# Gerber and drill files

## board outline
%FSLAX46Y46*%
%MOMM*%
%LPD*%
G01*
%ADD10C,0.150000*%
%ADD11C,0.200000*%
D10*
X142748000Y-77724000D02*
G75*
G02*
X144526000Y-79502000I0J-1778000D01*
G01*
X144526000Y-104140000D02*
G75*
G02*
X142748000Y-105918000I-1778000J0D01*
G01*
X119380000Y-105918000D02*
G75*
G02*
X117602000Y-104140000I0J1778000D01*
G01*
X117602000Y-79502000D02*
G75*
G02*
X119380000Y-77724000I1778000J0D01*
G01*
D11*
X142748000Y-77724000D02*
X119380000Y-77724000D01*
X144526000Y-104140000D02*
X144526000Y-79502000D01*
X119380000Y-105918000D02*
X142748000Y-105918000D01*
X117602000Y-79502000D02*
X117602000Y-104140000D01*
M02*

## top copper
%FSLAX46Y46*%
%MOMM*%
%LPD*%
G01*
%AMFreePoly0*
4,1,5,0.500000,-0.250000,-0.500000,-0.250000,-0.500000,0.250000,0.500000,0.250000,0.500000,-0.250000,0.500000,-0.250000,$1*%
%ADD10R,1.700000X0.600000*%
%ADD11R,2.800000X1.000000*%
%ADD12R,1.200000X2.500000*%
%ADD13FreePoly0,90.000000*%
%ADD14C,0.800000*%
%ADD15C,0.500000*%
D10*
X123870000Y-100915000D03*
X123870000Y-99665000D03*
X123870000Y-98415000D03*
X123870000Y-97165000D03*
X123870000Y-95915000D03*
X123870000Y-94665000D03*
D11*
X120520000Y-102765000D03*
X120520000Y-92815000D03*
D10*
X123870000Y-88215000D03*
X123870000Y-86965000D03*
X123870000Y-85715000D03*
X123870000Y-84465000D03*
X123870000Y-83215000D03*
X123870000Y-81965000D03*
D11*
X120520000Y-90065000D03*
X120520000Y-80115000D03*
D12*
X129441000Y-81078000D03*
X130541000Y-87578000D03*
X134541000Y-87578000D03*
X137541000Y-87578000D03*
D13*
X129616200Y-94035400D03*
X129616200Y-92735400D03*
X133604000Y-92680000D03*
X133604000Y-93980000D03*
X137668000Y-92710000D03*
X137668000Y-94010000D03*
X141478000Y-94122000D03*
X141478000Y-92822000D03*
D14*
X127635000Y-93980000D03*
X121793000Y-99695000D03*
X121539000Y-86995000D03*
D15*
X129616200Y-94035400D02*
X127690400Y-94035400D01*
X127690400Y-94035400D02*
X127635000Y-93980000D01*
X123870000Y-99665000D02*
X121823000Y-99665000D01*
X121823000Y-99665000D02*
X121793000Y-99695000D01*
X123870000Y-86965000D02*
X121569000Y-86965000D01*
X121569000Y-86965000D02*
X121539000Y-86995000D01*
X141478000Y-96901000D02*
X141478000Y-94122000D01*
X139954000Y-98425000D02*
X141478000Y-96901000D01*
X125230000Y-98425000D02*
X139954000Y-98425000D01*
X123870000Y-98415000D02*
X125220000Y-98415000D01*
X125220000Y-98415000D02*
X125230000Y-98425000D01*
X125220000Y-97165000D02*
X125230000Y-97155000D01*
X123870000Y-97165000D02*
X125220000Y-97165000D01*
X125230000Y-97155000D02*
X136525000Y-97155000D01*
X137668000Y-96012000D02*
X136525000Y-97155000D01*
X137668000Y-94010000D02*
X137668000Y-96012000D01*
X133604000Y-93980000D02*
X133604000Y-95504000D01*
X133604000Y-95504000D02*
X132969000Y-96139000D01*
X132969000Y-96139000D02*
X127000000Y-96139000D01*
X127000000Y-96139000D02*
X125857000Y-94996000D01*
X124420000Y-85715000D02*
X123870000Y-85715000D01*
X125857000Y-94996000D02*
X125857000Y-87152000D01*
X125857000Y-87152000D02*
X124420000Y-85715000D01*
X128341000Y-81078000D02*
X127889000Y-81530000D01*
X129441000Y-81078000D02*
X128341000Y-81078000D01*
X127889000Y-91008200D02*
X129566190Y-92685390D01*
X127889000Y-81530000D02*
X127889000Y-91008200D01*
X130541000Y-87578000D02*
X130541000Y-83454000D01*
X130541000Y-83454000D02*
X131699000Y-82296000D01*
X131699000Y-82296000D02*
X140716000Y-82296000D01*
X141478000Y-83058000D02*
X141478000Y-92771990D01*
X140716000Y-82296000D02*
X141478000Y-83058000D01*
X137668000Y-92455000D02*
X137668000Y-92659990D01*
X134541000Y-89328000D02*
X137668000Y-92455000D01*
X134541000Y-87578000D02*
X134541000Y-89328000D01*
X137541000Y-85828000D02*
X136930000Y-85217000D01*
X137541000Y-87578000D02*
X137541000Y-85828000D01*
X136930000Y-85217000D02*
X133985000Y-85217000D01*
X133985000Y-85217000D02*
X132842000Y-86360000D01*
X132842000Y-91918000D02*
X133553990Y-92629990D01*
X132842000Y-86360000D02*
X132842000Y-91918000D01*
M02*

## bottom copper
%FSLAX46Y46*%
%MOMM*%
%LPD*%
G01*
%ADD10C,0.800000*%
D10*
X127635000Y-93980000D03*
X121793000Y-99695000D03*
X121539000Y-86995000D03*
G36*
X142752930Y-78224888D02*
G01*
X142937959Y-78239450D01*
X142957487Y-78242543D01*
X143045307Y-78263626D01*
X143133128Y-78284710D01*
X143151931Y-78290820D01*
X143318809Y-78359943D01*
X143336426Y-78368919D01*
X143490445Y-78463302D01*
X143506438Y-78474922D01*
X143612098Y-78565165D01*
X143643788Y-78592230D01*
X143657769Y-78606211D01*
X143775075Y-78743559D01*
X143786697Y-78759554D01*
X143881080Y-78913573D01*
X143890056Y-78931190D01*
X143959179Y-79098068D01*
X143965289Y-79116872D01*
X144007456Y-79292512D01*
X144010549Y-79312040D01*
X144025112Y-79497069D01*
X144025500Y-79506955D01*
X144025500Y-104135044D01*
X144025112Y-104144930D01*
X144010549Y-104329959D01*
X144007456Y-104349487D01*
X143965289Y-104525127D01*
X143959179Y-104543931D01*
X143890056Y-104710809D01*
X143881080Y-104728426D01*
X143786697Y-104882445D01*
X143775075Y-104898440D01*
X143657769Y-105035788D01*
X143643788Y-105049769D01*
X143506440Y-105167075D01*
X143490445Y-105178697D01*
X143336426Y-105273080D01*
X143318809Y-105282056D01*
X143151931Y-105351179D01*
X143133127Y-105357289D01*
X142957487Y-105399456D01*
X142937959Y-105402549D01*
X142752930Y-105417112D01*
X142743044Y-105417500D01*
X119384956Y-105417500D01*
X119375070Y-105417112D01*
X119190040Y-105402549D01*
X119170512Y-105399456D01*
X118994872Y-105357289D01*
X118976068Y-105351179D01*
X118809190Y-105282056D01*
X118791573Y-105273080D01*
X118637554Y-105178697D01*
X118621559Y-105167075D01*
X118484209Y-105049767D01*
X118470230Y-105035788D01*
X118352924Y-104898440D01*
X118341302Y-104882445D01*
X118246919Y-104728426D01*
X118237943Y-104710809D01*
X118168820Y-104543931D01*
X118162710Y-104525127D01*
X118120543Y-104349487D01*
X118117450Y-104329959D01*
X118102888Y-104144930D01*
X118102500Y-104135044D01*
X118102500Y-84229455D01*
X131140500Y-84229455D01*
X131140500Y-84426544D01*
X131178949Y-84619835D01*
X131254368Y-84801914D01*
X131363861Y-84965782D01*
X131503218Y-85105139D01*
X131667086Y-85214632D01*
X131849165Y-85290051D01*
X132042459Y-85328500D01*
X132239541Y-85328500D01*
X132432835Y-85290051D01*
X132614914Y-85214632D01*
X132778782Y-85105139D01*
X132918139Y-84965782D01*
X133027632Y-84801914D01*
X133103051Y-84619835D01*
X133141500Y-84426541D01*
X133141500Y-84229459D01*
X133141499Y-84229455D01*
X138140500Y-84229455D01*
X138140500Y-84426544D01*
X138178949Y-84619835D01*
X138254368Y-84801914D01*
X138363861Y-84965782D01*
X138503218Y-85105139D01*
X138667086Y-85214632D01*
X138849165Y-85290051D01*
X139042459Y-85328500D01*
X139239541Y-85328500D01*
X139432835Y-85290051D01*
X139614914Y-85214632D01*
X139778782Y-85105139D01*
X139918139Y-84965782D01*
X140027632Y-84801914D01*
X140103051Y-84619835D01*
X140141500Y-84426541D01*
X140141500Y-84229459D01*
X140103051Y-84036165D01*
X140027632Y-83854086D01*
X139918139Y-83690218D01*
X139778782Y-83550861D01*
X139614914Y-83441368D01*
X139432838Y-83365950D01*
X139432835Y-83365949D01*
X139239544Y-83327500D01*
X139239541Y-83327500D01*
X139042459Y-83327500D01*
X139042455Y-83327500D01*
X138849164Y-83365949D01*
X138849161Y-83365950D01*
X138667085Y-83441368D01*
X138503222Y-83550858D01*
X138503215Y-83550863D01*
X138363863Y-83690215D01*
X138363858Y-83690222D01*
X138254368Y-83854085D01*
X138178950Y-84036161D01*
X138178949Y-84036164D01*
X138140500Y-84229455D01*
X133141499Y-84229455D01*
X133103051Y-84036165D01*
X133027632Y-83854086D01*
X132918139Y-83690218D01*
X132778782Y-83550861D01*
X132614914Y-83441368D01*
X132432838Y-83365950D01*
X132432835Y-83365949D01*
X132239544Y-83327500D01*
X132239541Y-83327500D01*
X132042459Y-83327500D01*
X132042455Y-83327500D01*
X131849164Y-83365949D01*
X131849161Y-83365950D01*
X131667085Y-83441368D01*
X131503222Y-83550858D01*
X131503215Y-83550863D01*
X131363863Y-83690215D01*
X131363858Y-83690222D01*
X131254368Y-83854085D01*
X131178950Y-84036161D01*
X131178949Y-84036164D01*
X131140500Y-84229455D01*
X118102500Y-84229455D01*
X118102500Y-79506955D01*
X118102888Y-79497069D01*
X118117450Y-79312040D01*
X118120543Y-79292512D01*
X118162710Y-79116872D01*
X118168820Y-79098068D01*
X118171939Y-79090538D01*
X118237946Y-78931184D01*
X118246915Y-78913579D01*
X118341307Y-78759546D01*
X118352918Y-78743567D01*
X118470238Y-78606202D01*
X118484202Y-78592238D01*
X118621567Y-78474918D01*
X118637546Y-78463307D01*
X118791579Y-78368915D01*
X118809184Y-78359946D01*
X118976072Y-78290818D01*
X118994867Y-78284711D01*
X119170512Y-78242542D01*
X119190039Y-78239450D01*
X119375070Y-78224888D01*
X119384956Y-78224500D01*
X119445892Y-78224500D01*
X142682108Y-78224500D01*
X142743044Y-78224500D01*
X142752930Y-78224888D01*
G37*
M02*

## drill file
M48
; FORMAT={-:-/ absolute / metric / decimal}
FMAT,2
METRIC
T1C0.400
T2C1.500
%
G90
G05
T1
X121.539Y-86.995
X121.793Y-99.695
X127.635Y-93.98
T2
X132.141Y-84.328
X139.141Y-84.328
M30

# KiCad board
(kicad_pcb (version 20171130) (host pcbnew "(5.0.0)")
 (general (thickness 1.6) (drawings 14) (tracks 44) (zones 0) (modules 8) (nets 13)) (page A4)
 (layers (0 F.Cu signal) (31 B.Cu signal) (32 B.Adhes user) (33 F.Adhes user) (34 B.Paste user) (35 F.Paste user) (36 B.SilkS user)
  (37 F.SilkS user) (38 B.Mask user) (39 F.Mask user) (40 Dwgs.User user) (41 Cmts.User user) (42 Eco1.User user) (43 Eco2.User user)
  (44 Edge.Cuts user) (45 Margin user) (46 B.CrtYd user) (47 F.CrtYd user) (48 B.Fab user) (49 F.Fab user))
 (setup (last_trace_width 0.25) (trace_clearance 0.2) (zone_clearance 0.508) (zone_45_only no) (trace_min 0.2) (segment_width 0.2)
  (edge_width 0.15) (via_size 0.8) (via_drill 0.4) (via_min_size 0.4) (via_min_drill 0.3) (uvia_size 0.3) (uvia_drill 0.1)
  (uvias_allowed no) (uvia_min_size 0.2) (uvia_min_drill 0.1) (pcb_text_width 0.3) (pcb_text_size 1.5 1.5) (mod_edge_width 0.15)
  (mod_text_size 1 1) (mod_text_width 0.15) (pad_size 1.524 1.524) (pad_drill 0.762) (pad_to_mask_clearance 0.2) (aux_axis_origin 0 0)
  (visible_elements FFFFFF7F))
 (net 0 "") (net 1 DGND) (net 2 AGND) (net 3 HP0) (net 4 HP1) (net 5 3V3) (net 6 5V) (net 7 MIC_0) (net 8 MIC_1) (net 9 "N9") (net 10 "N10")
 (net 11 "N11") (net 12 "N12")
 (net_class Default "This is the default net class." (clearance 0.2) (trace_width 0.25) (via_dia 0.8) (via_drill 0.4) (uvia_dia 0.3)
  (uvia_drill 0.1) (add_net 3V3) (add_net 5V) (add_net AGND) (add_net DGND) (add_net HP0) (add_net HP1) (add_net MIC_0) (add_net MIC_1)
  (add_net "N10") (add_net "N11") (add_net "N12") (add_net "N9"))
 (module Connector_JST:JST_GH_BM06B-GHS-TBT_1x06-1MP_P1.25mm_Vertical (layer F.Cu) (at 121.92 97.79 90)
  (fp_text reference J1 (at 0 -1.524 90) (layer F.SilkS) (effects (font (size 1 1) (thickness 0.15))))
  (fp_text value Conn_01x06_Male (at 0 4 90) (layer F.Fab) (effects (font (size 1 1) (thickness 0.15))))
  (pad 1 smd rect (at -3.125 1.95 90) (size 0.6 1.7) (layers F.Cu F.Paste F.Mask) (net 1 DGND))
  (pad 2 smd rect (at -1.875 1.95 90) (size 0.6 1.7) (layers F.Cu F.Paste F.Mask) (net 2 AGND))
  (pad 3 smd rect (at -0.625 1.95 90) (size 0.6 1.7) (layers F.Cu F.Paste F.Mask) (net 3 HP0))
  (pad 4 smd rect (at 0.625 1.95 90) (size 0.6 1.7) (layers F.Cu F.Paste F.Mask) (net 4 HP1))
  (pad 5 smd rect (at 1.875 1.95 90) (size 0.6 1.7) (layers F.Cu F.Paste F.Mask) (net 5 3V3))
  (pad 6 smd rect (at 3.125 1.95 90) (size 0.6 1.7) (layers F.Cu F.Paste F.Mask) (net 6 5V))
  (pad MP smd rect (at -4.975 -1.4 90) (size 1 2.8) (layers F.Cu F.Paste F.Mask))
  (pad MP smd rect (at 4.975 -1.4 90) (size 1 2.8) (layers F.Cu F.Paste F.Mask)))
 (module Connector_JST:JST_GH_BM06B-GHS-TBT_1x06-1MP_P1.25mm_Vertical (layer F.Cu) (at 121.92 85.09 90)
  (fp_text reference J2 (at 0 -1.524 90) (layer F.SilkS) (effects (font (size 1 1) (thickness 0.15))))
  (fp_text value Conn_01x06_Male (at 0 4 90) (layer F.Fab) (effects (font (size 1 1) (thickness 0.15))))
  (pad 1 smd rect (at -3.125 1.95 90) (size 0.6 1.7) (layers F.Cu F.Paste F.Mask) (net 1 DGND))
  (pad 2 smd rect (at -1.875 1.95 90) (size 0.6 1.7) (layers F.Cu F.Paste F.Mask) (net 2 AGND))
  (pad 3 smd rect (at -0.625 1.95 90) (size 0.6 1.7) (layers F.Cu F.Paste F.Mask) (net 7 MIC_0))
  (pad 4 smd rect (at 0.625 1.95 90) (size 0.6 1.7) (layers F.Cu F.Paste F.Mask) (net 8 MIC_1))
  (pad 5 smd rect (at 1.875 1.95 90) (size 0.6 1.7) (layers F.Cu F.Paste F.Mask) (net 5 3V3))
  (pad 6 smd rect (at 3.125 1.95 90) (size 0.6 1.7) (layers F.Cu F.Paste F.Mask) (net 6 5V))
  (pad MP smd rect (at -4.975 -1.4 90) (size 1 2.8) (layers F.Cu F.Paste F.Mask))
  (pad MP smd rect (at 4.975 -1.4 90) (size 1 2.8) (layers F.Cu F.Paste F.Mask)))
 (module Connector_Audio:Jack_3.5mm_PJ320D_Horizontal (layer F.Cu) (at 134.366 84.328 180)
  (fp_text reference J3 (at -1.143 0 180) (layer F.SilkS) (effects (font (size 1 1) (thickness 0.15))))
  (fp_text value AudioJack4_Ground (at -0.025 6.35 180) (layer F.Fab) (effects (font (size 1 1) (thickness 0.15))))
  (pad 4 smd rect (at 4.925 3.25 180) (size 1.2 2.5) (layers F.Cu F.Paste F.Mask) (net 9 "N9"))
  (pad 1 smd rect (at 3.825 -3.25 180) (size 1.2 2.5) (layers F.Cu F.Paste F.Mask) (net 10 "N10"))
  (pad 2 smd rect (at -0.175 -3.25 180) (size 1.2 2.5) (layers F.Cu F.Paste F.Mask) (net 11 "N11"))
  (pad 3 smd rect (at -3.175 -3.25 180) (size 1.2 2.5) (layers F.Cu F.Paste F.Mask) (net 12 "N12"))
  (pad "" np_thru_hole circle (at -4.775 0 180) (size 1.5 1.5) (drill 1.5) (layers *.Cu *.Mask))
  (pad "" np_thru_hole circle (at 2.225 0 180) (size 1.5 1.5) (drill 1.5) (layers *.Cu *.Mask)))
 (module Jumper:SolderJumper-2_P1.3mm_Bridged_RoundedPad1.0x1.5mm (layer F.Cu) (at 129.6162 93.3854 90)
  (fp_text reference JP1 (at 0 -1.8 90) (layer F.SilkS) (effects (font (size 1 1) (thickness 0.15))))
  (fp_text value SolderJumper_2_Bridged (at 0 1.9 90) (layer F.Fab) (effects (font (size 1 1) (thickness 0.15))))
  (pad 1 smd custom (at -0.65 0 90) (size 1 0.5) (layers F.Cu F.Mask) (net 2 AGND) (zone_connect 0)
   (options (clearance outline) (anchor rect)) (primitives))
  (pad 2 smd custom (at 0.65 0 90) (size 1 0.5) (layers F.Cu F.Mask) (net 9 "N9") (zone_connect 0)
   (options (clearance outline) (anchor rect)) (primitives)))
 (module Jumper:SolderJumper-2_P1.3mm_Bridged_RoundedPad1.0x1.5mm (layer F.Cu) (at 133.604 93.33 90)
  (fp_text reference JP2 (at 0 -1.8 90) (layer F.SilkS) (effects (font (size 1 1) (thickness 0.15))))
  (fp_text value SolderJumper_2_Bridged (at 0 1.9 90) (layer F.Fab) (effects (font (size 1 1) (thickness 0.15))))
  (pad 2 smd custom (at 0.65 0 90) (size 1 0.5) (layers F.Cu F.Mask) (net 12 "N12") (zone_connect 0)
   (options (clearance outline) (anchor rect)) (primitives))
  (pad 1 smd custom (at -0.65 0 90) (size 1 0.5) (layers F.Cu F.Mask) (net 7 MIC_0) (zone_connect 0)
   (options (clearance outline) (anchor rect)) (primitives)))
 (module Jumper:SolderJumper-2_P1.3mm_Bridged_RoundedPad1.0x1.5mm (layer F.Cu) (at 137.668 93.36 90)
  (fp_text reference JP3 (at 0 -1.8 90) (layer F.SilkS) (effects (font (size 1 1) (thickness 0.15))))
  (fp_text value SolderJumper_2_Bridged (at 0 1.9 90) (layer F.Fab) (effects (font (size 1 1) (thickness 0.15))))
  (pad 2 smd custom (at 0.65 0 90) (size 1 0.5) (layers F.Cu F.Mask) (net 11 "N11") (zone_connect 0)
   (options (clearance outline) (anchor rect)) (primitives))
  (pad 1 smd custom (at -0.65 0 90) (size 1 0.5) (layers F.Cu F.Mask) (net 4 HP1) (zone_connect 0)
   (options (clearance outline) (anchor rect)) (primitives)))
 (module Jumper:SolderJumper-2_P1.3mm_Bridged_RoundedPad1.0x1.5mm (layer F.Cu) (at 141.478 93.472 90)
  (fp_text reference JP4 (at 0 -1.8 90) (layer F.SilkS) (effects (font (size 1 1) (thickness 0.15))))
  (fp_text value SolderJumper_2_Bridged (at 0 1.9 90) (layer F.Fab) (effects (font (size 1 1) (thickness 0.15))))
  (pad 1 smd custom (at -0.65 0 90) (size 1 0.5) (layers F.Cu F.Mask) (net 3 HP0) (zone_connect 0)
   (options (clearance outline) (anchor rect)) (primitives))
  (pad 2 smd custom (at 0.65 0 90) (size 1 0.5) (layers F.Cu F.Mask) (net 10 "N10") (zone_connect 0)
   (options (clearance outline) (anchor rect)) (primitives)))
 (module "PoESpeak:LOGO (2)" (layer F.Cu) (at 135.128 102.616)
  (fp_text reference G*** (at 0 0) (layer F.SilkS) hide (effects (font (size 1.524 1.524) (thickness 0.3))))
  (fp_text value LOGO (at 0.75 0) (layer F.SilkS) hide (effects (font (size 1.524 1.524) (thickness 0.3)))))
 (gr_arc (start 142.748 79.502) (end 144.526 79.502) (angle -90) (layer Edge.Cuts) (width 0.15))
 (gr_arc (start 142.748 104.14) (end 142.748 105.918) (angle -90) (layer Edge.Cuts) (width 0.15))
 (gr_arc (start 119.38 104.14) (end 117.602 104.14) (angle -90) (layer Edge.Cuts) (width 0.15))
 (gr_arc (start 119.38 79.502) (end 119.38 77.724) (angle -90) (layer Edge.Cuts) (width 0.15))
 (gr_line (start 142.748 77.724) (end 119.38 77.724) (layer Edge.Cuts) (width 0.2))
 (gr_line (start 144.526 104.14) (end 144.526 79.502) (layer Edge.Cuts) (width 0.2))
 (gr_line (start 119.38 105.918) (end 142.748 105.918) (layer Edge.Cuts) (width 0.2))
 (gr_line (start 117.602 79.502) (end 117.602 104.14) (layer Edge.Cuts) (width 0.2))
 (via (at 127.635 93.98) (size 0.8) (drill 0.4) (layers F.Cu B.Cu) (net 2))
 (segment (start 129.6162 94.0354) (end 127.6904 94.0354) (width 0.5) (layer F.Cu) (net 2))
 (segment (start 127.6904 94.0354) (end 127.635 93.98) (width 0.5) (layer F.Cu) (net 2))
 (via (at 121.793 99.695) (size 0.8) (drill 0.4) (layers F.Cu B.Cu) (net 2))
 (segment (start 123.87 99.665) (end 121.823 99.665) (width 0.5) (layer F.Cu) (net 2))
 (segment (start 121.823 99.665) (end 121.793 99.695) (width 0.5) (layer F.Cu) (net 2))
 (via (at 121.539 86.995) (size 0.8) (drill 0.4) (layers F.Cu B.Cu) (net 2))
 (segment (start 123.87 86.965) (end 121.569 86.965) (width 0.5) (layer F.Cu) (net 2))
 (segment (start 121.569 86.965) (end 121.539 86.995) (width 0.5) (layer F.Cu) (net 2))
 (segment (start 141.478 96.901) (end 141.478 94.122) (width 0.5) (layer F.Cu) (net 3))
 (segment (start 139.954 98.425) (end 141.478 96.901) (width 0.5) (layer F.Cu) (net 3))
 (segment (start 125.23 98.425) (end 139.954 98.425) (width 0.5) (layer F.Cu) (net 3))
 (segment (start 123.87 98.415) (end 125.22 98.415) (width 0.5) (layer F.Cu) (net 3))
 (segment (start 125.22 98.415) (end 125.23 98.425) (width 0.5) (layer F.Cu) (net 3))
 (segment (start 125.22 97.165) (end 125.23 97.155) (width 0.5) (layer F.Cu) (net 4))
 (segment (start 123.87 97.165) (end 125.22 97.165) (width 0.5) (layer F.Cu) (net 4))
 (segment (start 125.23 97.155) (end 136.525 97.155) (width 0.5) (layer F.Cu) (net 4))
 (segment (start 137.668 96.012) (end 136.525 97.155) (width 0.5) (layer F.Cu) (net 4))
 (segment (start 137.668 94.01) (end 137.668 96.012) (width 0.5) (layer F.Cu) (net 4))
 (segment (start 133.604 93.98) (end 133.604 95.504) (width 0.5) (layer F.Cu) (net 7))
 (segment (start 133.604 95.504) (end 132.969 96.139) (width 0.5) (layer F.Cu) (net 7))
 (segment (start 132.969 96.139) (end 127 96.139) (width 0.5) (layer F.Cu) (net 7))
 (segment (start 127 96.139) (end 125.857 94.996) (width 0.5) (layer F.Cu) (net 7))
 (segment (start 124.42 85.715) (end 123.87 85.715) (width 0.5) (layer F.Cu) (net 7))
 (segment (start 125.857 94.996) (end 125.857 87.152) (width 0.5) (layer F.Cu) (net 7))
 (segment (start 125.857 87.152) (end 124.42 85.715) (width 0.5) (layer F.Cu) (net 7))
 (segment (start 128.341 81.078) (end 127.889 81.53) (width 0.5) (layer F.Cu) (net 9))
 (segment (start 129.441 81.078) (end 128.341 81.078) (width 0.5) (layer F.Cu) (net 9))
 (segment (start 127.889 91.0082) (end 129.56619 92.68539) (width 0.5) (layer F.Cu) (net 9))
 (segment (start 127.889 81.53) (end 127.889 91.0082) (width 0.5) (layer F.Cu) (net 9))
 (segment (start 130.541 87.578) (end 130.541 83.454) (width 0.5) (layer F.Cu) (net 10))
 (segment (start 130.541 83.454) (end 131.699 82.296) (width 0.5) (layer F.Cu) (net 10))
 (segment (start 131.699 82.296) (end 140.716 82.296) (width 0.5) (layer F.Cu) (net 10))
 (segment (start 141.478 83.058) (end 141.478 92.77199) (width 0.5) (layer F.Cu) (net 10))
 (segment (start 140.716 82.296) (end 141.478 83.058) (width 0.5) (layer F.Cu) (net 10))
 (segment (start 137.668 92.455) (end 137.668 92.65999) (width 0.5) (layer F.Cu) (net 11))
 (segment (start 134.541 89.328) (end 137.668 92.455) (width 0.5) (layer F.Cu) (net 11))
 (segment (start 134.541 87.578) (end 134.541 89.328) (width 0.5) (layer F.Cu) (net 11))
 (segment (start 137.541 85.828) (end 136.93 85.217) (width 0.5) (layer F.Cu) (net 12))
 (segment (start 137.541 87.578) (end 137.541 85.828) (width 0.5) (layer F.Cu) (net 12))
 (segment (start 136.93 85.217) (end 133.985 85.217) (width 0.5) (layer F.Cu) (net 12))
 (segment (start 133.985 85.217) (end 132.842 86.36) (width 0.5) (layer F.Cu) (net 12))
 (segment (start 132.842 91.918) (end 133.55399 92.62999) (width 0.5) (layer F.Cu) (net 12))
 (segment (start 132.842 86.36) (end 132.842 91.918) (width 0.5) (layer F.Cu) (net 12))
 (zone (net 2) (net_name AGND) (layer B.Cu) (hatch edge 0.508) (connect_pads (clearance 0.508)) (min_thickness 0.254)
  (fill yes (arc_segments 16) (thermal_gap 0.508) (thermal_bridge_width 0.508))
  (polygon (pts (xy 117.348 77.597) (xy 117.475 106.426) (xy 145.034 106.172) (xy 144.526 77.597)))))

